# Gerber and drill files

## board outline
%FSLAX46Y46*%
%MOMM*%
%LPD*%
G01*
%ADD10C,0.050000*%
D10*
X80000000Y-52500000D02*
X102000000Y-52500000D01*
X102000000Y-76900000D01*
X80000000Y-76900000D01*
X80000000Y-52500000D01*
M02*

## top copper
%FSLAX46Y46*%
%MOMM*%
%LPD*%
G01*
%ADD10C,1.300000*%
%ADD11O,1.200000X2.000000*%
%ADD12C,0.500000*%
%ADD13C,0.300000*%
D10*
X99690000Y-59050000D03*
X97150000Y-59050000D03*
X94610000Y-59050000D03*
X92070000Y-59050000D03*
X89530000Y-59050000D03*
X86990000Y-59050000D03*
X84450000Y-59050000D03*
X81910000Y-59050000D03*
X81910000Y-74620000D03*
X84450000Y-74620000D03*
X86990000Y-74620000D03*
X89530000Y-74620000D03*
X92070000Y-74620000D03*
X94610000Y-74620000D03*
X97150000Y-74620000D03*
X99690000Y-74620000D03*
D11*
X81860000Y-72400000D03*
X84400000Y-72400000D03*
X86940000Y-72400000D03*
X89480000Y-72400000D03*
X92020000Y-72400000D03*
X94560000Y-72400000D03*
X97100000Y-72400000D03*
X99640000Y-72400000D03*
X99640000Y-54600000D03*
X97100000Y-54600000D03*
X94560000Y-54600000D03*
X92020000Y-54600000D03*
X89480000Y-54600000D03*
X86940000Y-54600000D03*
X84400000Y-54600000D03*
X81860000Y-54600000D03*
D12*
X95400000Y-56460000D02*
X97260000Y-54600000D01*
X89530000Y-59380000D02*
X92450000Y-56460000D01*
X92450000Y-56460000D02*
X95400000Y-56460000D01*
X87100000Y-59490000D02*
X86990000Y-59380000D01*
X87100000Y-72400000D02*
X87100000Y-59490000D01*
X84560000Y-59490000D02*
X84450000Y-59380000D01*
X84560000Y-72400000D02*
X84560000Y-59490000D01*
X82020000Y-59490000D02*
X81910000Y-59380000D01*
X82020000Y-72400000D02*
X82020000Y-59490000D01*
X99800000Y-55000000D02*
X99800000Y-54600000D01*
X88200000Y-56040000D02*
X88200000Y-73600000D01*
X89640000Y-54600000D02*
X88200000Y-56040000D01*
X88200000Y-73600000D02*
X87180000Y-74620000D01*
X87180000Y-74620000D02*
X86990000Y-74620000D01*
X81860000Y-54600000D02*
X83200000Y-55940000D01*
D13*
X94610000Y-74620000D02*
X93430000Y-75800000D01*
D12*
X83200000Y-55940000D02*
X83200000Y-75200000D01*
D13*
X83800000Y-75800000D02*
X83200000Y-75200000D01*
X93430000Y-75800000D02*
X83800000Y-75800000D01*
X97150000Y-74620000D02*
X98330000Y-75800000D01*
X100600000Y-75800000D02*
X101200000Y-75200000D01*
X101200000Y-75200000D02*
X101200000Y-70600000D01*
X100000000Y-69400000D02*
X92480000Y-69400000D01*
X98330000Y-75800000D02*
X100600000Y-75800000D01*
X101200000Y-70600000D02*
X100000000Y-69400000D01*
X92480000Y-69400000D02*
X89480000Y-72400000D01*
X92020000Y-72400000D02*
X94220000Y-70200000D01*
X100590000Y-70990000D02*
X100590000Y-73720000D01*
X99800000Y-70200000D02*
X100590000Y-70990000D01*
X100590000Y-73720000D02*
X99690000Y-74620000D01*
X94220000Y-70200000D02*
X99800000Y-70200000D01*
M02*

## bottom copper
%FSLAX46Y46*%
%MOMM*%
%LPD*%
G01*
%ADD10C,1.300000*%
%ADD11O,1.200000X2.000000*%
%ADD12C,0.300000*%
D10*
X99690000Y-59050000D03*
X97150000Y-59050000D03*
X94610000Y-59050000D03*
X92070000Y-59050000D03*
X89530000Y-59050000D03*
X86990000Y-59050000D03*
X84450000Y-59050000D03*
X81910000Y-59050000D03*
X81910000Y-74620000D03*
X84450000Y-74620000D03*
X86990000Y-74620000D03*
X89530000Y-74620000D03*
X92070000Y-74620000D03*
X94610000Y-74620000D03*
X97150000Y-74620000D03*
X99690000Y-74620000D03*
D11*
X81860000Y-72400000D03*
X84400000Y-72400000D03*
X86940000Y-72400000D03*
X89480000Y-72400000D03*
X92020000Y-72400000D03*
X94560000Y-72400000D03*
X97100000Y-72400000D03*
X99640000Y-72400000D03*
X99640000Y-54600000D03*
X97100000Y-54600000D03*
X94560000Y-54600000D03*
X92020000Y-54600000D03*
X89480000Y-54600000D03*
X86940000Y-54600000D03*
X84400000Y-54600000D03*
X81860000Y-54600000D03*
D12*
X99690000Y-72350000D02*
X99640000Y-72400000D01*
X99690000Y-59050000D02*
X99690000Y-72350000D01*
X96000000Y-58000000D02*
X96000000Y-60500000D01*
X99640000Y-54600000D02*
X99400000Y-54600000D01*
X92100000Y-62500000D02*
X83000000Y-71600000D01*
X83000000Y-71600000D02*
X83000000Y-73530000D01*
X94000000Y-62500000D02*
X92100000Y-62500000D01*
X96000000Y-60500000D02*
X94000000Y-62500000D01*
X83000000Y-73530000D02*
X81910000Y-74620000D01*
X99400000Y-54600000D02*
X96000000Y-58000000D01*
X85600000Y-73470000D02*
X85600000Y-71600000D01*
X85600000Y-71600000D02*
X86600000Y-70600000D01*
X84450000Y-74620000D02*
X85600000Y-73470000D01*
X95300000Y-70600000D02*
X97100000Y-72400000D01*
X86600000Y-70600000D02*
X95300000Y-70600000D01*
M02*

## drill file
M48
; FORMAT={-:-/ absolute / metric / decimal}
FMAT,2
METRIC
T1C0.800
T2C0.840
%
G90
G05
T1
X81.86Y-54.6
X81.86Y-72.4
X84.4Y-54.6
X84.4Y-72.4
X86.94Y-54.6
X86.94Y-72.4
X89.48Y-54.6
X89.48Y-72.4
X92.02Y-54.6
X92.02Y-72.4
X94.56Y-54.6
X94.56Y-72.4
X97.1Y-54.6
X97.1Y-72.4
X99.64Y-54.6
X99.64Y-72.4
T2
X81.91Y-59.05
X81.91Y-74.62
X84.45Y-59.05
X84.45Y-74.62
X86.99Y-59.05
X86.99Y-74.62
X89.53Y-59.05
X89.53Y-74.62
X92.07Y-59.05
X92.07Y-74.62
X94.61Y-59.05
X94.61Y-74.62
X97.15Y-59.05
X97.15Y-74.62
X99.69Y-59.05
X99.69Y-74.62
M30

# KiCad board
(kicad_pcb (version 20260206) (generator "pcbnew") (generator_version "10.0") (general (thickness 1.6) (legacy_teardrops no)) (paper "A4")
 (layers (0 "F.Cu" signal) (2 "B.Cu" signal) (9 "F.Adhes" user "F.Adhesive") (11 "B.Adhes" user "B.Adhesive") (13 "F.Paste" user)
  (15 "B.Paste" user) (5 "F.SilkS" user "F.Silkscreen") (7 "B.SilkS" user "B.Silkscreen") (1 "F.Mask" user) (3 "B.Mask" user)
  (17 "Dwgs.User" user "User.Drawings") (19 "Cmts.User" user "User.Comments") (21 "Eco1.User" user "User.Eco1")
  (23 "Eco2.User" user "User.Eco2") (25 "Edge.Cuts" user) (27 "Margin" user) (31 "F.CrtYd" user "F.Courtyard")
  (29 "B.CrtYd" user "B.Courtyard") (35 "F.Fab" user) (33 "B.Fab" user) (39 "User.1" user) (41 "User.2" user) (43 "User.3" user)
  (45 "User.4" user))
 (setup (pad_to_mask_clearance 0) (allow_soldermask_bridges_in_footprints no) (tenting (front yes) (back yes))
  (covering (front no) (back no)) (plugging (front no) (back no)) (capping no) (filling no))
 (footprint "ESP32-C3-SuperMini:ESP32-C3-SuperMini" (layer "F.Cu") (at 90.8 67 90)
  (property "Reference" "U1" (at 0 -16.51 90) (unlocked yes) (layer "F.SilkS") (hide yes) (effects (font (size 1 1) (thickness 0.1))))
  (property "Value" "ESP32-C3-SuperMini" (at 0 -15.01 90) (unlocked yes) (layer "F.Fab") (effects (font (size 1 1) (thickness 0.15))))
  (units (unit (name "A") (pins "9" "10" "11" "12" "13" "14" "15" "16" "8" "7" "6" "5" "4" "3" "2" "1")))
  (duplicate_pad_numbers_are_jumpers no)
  (pad "1" thru_hole circle (at 7.95 8.89 90) (size 1.3 1.3) (drill 0.84) (layers "*.Cu" "*.Mask") (remove_unused_layers no)
   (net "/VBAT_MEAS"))
  (pad "2" thru_hole circle (at 7.95 6.35 90) (size 1.3 1.3) (drill 0.84) (layers "*.Cu" "*.Mask") (remove_unused_layers no)
   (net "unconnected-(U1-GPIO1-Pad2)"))
  (pad "3" thru_hole circle (at 7.95 3.81 90) (size 1.3 1.3) (drill 0.84) (layers "*.Cu" "*.Mask") (remove_unused_layers no)
   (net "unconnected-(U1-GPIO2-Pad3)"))
  (pad "4" thru_hole circle (at 7.95 1.27 90) (size 1.3 1.3) (drill 0.84) (layers "*.Cu" "*.Mask") (remove_unused_layers no)
   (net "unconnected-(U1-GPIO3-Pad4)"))
  (pad "5" thru_hole circle (at 7.95 -1.27 90) (size 1.3 1.3) (drill 0.84) (layers "*.Cu" "*.Mask") (remove_unused_layers no)
   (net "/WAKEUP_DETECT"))
  (pad "6" thru_hole circle (at 7.95 -3.81 90) (size 1.3 1.3) (drill 0.84) (layers "*.Cu" "*.Mask") (remove_unused_layers no) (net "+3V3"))
  (pad "7" thru_hole circle (at 7.95 -6.35 90) (size 1.3 1.3) (drill 0.84) (layers "*.Cu" "*.Mask") (remove_unused_layers no) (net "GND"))
  (pad "8" thru_hole circle (at 7.95 -8.89 90) (size 1.3 1.3) (drill 0.84) (layers "*.Cu" "*.Mask") (remove_unused_layers no) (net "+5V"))
  (pad "9" thru_hole circle (at -7.62 -8.89 90) (size 1.3 1.3) (drill 0.84) (layers "*.Cu" "*.Mask") (remove_unused_layers no)
   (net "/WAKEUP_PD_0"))
  (pad "10" thru_hole circle (at -7.62 -6.35 90) (size 1.3 1.3) (drill 0.84) (layers "*.Cu" "*.Mask") (remove_unused_layers no)
   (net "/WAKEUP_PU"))
  (pad "11" thru_hole circle (at -7.62 -3.81 90) (size 1.3 1.3) (drill 0.84) (layers "*.Cu" "*.Mask") (remove_unused_layers no)
   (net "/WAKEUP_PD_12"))
  (pad "12" thru_hole circle (at -7.62 -1.27 90) (size 1.3 1.3) (drill 0.84) (layers "*.Cu" "*.Mask") (remove_unused_layers no)
   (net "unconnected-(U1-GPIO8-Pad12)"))
  (pad "13" thru_hole circle (at -7.62 1.27 90) (size 1.3 1.3) (drill 0.84) (layers "*.Cu" "*.Mask") (remove_unused_layers no)
   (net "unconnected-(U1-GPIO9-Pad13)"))
  (pad "14" thru_hole circle (at -7.62 3.81 90) (size 1.3 1.3) (drill 0.84) (layers "*.Cu" "*.Mask") (remove_unused_layers no)
   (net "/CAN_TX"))
  (pad "15" thru_hole circle (at -7.62 6.35 90) (size 1.3 1.3) (drill 0.84) (layers "*.Cu" "*.Mask") (remove_unused_layers no)
   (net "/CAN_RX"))
  (pad "16" thru_hole circle (at -7.62 8.89 90) (size 1.3 1.3) (drill 0.84) (layers "*.Cu" "*.Mask") (remove_unused_layers no)
   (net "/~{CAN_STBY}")))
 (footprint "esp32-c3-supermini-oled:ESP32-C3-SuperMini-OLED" (layer "F.Cu") (at 90.75 63.5)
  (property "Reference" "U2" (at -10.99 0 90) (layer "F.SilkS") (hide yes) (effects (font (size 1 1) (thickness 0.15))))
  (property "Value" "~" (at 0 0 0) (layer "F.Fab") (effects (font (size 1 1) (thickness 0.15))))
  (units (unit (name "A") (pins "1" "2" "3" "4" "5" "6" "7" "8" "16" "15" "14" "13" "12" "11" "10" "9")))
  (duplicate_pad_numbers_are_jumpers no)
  (pad "1" thru_hole oval (at -8.89 8.9) (size 1.2 2) (drill 0.8) (layers "*.Cu" "*.Mask") (remove_unused_layers no) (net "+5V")
   (thermal_bridge_angle 45))
  (pad "2" thru_hole oval (at -6.35 8.9) (size 1.2 2) (drill 0.8) (layers "*.Cu" "*.Mask") (remove_unused_layers no) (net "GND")
   (thermal_bridge_angle 45))
  (pad "3" thru_hole oval (at -3.81 8.9) (size 1.2 2) (drill 0.8) (layers "*.Cu" "*.Mask") (remove_unused_layers no) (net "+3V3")
   (thermal_bridge_angle 45))
  (pad "4" thru_hole oval (at -1.27 8.9) (size 1.2 2) (drill 0.8) (layers "*.Cu" "*.Mask") (remove_unused_layers no) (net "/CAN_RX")
   (thermal_bridge_angle 45))
  (pad "5" thru_hole oval (at 1.27 8.9) (size 1.2 2) (drill 0.8) (layers "*.Cu" "*.Mask") (remove_unused_layers no) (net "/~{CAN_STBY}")
   (thermal_bridge_angle 45))
  (pad "6" thru_hole oval (at 3.81 8.9) (size 1.2 2) (drill 0.8) (layers "*.Cu" "*.Mask") (remove_unused_layers no)
   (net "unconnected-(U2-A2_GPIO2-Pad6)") (thermal_bridge_angle 45))
  (pad "7" thru_hole oval (at 6.35 8.9) (size 1.2 2) (drill 0.8) (layers "*.Cu" "*.Mask") (remove_unused_layers no) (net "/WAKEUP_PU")
   (thermal_bridge_angle 45))
  (pad "8" thru_hole oval (at 8.89 8.9) (size 1.2 2) (drill 0.8) (layers "*.Cu" "*.Mask") (remove_unused_layers no) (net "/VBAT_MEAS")
   (thermal_bridge_angle 45))
  (pad "9" thru_hole oval (at 8.89 -8.9) (size 1.2 2) (drill 0.8) (layers "*.Cu" "*.Mask") (remove_unused_layers no) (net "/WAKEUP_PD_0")
   (thermal_bridge_angle 45))
  (pad "10" thru_hole oval (at 6.35 -8.9) (size 1.2 2) (drill 0.8) (layers "*.Cu" "*.Mask") (remove_unused_layers no) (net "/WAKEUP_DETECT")
   (thermal_bridge_angle 45))
  (pad "11" thru_hole oval (at 3.81 -8.9) (size 1.2 2) (drill 0.8) (layers "*.Cu" "*.Mask") (remove_unused_layers no)
   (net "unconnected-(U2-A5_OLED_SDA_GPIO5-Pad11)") (thermal_bridge_angle 45))
  (pad "12" thru_hole oval (at 1.27 -8.9) (size 1.2 2) (drill 0.8) (layers "*.Cu" "*.Mask") (remove_unused_layers no)
   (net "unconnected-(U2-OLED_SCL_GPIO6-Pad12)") (thermal_bridge_angle 45))
  (pad "13" thru_hole oval (at -1.27 -8.9) (size 1.2 2) (drill 0.8) (layers "*.Cu" "*.Mask") (remove_unused_layers no) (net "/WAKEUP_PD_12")
   (thermal_bridge_angle 45))
  (pad "14" thru_hole oval (at -3.81 -8.9) (size 1.2 2) (drill 0.8) (layers "*.Cu" "*.Mask") (remove_unused_layers no)
   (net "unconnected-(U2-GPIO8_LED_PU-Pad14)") (thermal_bridge_angle 45))
  (pad "15" thru_hole oval (at -6.35 -8.9) (size 1.2 2) (drill 0.8) (layers "*.Cu" "*.Mask") (remove_unused_layers no)
   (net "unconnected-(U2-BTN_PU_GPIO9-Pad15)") (thermal_bridge_angle 45))
  (pad "16" thru_hole oval (at -8.89 -8.9) (size 1.2 2) (drill 0.8) (layers "*.Cu" "*.Mask") (remove_unused_layers no) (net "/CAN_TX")
   (thermal_bridge_angle 45)))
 (gr_rect (start 80 52.5) (end 102 76.9) (stroke (width 0.05) (type default)) (fill no) (layer "Edge.Cuts"))
 (segment (start 99.69 72.35) (end 99.64 72.4) (width 0.3) (layer "B.Cu") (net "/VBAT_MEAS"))
 (segment (start 99.69 59.05) (end 99.69 72.35) (width 0.3) (layer "B.Cu") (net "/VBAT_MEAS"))
 (segment (start 95.4 56.46) (end 97.26 54.6) (width 0.5) (layer "F.Cu") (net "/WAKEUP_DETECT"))
 (segment (start 89.53 59.38) (end 92.45 56.46) (width 0.5) (layer "F.Cu") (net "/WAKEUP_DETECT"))
 (segment (start 92.45 56.46) (end 95.4 56.46) (width 0.5) (layer "F.Cu") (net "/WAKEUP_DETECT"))
 (segment (start 87.1 59.49) (end 86.99 59.38) (width 0.5) (layer "F.Cu") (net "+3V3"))
 (segment (start 87.1 72.4) (end 87.1 59.49) (width 0.5) (layer "F.Cu") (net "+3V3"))
 (segment (start 84.56 59.49) (end 84.45 59.38) (width 0.5) (layer "F.Cu") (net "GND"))
 (segment (start 84.56 72.4) (end 84.56 59.49) (width 0.5) (layer "F.Cu") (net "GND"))
 (segment (start 82.02 59.49) (end 81.91 59.38) (width 0.5) (layer "F.Cu") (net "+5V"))
 (segment (start 82.02 72.4) (end 82.02 59.49) (width 0.5) (layer "F.Cu") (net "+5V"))
 (segment (start 99.8 55) (end 99.8 54.6) (width 0.5) (layer "F.Cu") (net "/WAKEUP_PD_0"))
 (segment (start 96 58) (end 96 60.5) (width 0.3) (layer "B.Cu") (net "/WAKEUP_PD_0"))
 (segment (start 99.64 54.6) (end 99.4 54.6) (width 0.3) (layer "B.Cu") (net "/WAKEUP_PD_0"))
 (segment (start 92.1 62.5) (end 83 71.6) (width 0.3) (layer "B.Cu") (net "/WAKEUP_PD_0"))
 (segment (start 83 71.6) (end 83 73.53) (width 0.3) (layer "B.Cu") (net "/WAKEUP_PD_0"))
 (segment (start 94 62.5) (end 92.1 62.5) (width 0.3) (layer "B.Cu") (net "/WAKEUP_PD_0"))
 (segment (start 96 60.5) (end 94 62.5) (width 0.3) (layer "B.Cu") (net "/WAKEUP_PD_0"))
 (segment (start 83 73.53) (end 81.91 74.62) (width 0.3) (layer "B.Cu") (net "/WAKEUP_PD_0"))
 (segment (start 99.4 54.6) (end 96 58) (width 0.3) (layer "B.Cu") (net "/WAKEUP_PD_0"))
 (segment (start 85.6 73.47) (end 85.6 71.6) (width 0.3) (layer "B.Cu") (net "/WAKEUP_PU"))
 (segment (start 85.6 71.6) (end 86.6 70.6) (width 0.3) (layer "B.Cu") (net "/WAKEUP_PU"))
 (segment (start 84.45 74.62) (end 85.6 73.47) (width 0.3) (layer "B.Cu") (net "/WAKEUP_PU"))
 (segment (start 95.3 70.6) (end 97.1 72.4) (width 0.3) (layer "B.Cu") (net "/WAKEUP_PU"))
 (segment (start 86.6 70.6) (end 95.3 70.6) (width 0.3) (layer "B.Cu") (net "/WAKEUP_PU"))
 (segment (start 88.2 56.04) (end 88.2 73.6) (width 0.5) (layer "F.Cu") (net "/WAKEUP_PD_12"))
 (segment (start 89.64 54.6) (end 88.2 56.04) (width 0.5) (layer "F.Cu") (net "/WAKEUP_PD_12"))
 (segment (start 88.2 73.6) (end 87.18 74.62) (width 0.5) (layer "F.Cu") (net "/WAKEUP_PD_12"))
 (segment (start 87.18 74.62) (end 86.99 74.62) (width 0.5) (layer "F.Cu") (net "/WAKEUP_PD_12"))
 (segment (start 81.86 54.6) (end 83.2 55.94) (width 0.5) (layer "F.Cu") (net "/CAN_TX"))
 (segment (start 94.61 74.62) (end 93.43 75.8) (width 0.3) (layer "F.Cu") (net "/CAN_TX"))
 (segment (start 83.2 55.94) (end 83.2 75.2) (width 0.5) (layer "F.Cu") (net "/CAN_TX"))
 (segment (start 83.8 75.8) (end 83.2 75.2) (width 0.3) (layer "F.Cu") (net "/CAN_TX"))
 (segment (start 93.43 75.8) (end 83.8 75.8) (width 0.3) (layer "F.Cu") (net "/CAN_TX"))
 (segment (start 97.15 74.62) (end 98.33 75.8) (width 0.3) (layer "F.Cu") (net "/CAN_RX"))
 (segment (start 100.6 75.8) (end 101.2 75.2) (width 0.3) (layer "F.Cu") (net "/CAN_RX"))
 (segment (start 101.2 75.2) (end 101.2 70.6) (width 0.3) (layer "F.Cu") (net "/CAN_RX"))
 (segment (start 100 69.4) (end 92.48 69.4) (width 0.3) (layer "F.Cu") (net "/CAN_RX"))
 (segment (start 98.33 75.8) (end 100.6 75.8) (width 0.3) (layer "F.Cu") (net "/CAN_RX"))
 (segment (start 101.2 70.6) (end 100 69.4) (width 0.3) (layer "F.Cu") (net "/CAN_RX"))
 (segment (start 92.48 69.4) (end 89.48 72.4) (width 0.3) (layer "F.Cu") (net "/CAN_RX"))
 (segment (start 92.02 72.4) (end 94.22 70.2) (width 0.3) (layer "F.Cu") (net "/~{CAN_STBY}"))
 (segment (start 100.59 70.99) (end 100.59 73.72) (width 0.3) (layer "F.Cu") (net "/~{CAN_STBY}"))
 (segment (start 99.8 70.2) (end 100.59 70.99) (width 0.3) (layer "F.Cu") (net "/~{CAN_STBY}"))
 (segment (start 100.59 73.72) (end 99.69 74.62) (width 0.3) (layer "F.Cu") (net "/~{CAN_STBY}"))
 (segment (start 94.22 70.2) (end 99.8 70.2) (width 0.3) (layer "F.Cu") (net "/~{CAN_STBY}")))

